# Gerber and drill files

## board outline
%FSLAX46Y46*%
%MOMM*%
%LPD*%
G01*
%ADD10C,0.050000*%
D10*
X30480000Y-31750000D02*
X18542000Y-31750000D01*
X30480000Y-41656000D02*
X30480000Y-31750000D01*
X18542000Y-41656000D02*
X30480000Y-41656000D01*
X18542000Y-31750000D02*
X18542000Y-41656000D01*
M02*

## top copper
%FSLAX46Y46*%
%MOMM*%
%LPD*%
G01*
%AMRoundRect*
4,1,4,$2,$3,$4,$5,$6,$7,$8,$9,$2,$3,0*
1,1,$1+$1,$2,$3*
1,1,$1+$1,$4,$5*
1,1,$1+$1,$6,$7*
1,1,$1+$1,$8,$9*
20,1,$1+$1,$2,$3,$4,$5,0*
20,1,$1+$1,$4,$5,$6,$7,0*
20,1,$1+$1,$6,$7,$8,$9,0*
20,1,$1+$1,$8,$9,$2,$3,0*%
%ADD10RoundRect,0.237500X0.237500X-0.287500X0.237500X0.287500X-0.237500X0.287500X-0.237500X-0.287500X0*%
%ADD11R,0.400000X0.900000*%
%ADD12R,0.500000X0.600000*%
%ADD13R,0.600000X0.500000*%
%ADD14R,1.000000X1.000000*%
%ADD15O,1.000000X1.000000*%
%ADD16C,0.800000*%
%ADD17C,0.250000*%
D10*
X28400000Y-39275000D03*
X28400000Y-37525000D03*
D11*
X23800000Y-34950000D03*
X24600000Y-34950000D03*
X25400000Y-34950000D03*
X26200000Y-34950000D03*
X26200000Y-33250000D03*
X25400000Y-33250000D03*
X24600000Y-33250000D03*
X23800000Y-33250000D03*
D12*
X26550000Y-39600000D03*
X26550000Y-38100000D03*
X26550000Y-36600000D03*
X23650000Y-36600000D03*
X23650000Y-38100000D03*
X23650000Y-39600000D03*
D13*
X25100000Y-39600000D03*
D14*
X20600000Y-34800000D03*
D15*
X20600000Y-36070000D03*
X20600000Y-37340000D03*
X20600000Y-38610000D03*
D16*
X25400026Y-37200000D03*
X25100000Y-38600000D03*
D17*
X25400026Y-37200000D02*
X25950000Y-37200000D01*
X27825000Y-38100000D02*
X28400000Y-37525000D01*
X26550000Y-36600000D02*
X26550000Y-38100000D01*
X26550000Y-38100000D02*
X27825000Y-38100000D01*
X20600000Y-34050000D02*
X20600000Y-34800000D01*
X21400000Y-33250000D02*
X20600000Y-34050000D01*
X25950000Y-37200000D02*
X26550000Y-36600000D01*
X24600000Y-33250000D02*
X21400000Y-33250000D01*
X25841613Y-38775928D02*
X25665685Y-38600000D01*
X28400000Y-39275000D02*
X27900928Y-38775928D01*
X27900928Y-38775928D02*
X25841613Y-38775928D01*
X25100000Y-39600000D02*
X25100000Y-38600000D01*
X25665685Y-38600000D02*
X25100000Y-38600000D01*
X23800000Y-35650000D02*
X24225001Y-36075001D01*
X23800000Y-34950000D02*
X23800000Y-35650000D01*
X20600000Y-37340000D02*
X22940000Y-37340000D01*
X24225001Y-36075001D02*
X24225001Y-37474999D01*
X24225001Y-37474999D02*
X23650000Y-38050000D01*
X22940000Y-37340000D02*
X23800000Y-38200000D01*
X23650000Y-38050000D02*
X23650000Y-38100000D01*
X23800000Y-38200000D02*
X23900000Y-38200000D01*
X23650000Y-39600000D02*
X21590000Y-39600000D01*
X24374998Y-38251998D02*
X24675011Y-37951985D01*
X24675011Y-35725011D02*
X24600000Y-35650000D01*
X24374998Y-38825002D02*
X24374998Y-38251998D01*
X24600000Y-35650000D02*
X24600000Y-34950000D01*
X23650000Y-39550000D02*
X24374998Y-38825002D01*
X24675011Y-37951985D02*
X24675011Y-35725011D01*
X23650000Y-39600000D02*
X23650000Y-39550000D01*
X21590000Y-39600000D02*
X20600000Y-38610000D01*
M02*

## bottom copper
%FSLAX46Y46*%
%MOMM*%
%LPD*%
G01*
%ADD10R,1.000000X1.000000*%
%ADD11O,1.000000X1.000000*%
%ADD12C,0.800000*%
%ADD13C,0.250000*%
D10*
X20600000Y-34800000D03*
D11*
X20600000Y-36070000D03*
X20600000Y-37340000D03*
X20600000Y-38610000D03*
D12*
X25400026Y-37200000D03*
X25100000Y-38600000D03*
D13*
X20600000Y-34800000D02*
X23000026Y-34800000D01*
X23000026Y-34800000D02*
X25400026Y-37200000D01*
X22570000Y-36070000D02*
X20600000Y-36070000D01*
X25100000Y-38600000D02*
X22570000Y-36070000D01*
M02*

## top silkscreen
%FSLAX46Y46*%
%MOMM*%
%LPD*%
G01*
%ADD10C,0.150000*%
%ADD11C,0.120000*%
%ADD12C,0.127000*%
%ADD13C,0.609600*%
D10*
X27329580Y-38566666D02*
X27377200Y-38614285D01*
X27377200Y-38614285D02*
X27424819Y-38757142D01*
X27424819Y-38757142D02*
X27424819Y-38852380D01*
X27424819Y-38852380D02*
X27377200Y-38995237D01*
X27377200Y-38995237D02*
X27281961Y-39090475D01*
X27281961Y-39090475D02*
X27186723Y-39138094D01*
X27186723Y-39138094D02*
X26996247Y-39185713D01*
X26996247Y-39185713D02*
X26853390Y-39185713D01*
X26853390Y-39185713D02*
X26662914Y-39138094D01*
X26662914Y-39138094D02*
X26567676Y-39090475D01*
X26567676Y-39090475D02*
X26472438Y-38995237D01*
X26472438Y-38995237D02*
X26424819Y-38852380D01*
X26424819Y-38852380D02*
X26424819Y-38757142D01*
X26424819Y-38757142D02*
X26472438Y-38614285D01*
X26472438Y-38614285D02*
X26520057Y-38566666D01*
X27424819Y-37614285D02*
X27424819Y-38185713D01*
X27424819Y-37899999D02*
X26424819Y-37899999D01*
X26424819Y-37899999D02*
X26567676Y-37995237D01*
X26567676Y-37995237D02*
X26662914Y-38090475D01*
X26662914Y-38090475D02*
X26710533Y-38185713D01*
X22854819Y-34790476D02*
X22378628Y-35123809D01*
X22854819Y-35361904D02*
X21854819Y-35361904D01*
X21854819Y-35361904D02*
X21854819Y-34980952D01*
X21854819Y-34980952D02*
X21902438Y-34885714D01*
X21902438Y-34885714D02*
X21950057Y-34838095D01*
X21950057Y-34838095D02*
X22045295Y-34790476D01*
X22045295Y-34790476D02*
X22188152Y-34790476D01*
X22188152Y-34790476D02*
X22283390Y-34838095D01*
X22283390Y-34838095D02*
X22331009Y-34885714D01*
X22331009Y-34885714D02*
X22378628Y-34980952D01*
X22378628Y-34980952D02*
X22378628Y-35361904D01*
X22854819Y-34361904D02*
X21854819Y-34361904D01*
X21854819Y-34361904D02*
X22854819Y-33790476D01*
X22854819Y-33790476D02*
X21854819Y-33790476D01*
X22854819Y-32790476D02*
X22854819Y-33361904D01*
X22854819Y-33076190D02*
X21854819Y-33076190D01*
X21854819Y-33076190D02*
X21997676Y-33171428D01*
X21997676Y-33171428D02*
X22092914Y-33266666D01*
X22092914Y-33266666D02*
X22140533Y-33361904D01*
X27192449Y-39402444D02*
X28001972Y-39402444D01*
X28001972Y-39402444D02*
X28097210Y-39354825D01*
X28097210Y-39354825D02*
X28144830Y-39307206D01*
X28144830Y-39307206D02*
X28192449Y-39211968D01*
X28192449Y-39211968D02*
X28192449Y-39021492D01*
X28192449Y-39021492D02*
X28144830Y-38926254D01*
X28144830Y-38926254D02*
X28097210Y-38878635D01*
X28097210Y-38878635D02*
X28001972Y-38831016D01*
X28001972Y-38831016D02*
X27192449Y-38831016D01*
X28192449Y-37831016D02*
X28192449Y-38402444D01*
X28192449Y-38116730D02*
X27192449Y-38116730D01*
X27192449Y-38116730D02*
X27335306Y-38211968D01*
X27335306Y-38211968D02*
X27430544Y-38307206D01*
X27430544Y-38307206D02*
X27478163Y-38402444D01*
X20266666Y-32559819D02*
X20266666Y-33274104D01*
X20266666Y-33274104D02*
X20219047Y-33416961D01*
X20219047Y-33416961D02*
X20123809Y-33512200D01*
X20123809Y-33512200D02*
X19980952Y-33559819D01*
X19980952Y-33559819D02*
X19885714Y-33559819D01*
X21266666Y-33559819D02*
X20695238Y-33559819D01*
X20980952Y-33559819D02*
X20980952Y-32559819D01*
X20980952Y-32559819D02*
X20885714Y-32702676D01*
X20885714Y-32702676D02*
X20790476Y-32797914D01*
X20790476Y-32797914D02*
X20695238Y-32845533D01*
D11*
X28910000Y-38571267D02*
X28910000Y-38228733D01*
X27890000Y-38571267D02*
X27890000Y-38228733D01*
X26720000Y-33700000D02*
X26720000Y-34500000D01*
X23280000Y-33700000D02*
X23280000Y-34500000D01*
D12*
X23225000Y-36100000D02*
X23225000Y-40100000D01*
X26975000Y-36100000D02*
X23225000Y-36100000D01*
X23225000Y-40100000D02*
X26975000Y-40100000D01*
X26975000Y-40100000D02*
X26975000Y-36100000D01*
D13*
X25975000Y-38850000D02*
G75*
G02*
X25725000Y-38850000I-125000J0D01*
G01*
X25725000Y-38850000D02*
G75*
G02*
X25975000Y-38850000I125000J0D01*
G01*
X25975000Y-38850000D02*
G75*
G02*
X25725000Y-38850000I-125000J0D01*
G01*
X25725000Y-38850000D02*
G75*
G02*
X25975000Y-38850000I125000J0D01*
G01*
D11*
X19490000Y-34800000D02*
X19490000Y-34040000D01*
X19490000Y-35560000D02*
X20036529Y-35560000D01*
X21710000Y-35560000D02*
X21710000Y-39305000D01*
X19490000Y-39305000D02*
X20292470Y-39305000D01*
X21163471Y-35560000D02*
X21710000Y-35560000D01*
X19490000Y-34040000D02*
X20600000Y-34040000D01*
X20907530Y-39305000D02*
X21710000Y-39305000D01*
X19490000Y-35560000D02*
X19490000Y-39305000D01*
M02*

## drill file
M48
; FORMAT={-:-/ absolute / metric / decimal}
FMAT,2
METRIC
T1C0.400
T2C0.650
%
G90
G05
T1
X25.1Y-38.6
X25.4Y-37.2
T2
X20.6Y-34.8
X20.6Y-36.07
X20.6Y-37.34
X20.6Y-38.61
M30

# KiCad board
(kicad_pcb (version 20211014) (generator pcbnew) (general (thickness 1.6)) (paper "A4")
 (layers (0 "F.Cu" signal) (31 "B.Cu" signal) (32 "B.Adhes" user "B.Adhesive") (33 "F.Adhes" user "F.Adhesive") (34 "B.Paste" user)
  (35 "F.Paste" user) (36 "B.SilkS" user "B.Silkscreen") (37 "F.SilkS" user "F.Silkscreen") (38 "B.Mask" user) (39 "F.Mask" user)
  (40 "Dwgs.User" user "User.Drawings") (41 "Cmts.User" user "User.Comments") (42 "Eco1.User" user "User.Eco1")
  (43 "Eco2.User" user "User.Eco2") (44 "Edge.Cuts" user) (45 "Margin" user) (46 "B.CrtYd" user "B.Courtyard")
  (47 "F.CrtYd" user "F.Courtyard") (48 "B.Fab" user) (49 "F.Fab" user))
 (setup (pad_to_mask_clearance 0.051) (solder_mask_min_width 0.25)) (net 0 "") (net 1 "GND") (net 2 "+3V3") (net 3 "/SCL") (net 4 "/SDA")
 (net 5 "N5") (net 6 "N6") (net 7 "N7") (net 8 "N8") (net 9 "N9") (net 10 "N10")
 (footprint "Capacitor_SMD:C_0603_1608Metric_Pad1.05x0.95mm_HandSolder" (layer "F.Cu") (at 28.4 38.4 90)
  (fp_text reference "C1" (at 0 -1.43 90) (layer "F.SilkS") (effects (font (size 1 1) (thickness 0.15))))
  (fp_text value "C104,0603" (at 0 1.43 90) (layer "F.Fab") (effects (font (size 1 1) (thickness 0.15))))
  (fp_line (start -0.171267 0.51) (end 0.171267 0.51) (layer "F.SilkS") (width 0.12))
  (fp_line (start -0.171267 -0.51) (end 0.171267 -0.51) (layer "F.SilkS") (width 0.12))
  (pad "1" smd roundrect locked (at -0.875 0 90) (size 1.05 0.95) (layers "F.Cu" "F.Paste" "F.Mask") (roundrect_rratio 0.25) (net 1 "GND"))
  (pad "2" smd roundrect locked (at 0.875 0 90) (size 1.05 0.95) (layers "F.Cu" "F.Paste" "F.Mask") (roundrect_rratio 0.25) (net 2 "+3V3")))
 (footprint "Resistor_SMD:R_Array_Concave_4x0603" (layer "F.Cu") (at 25 34.1 90)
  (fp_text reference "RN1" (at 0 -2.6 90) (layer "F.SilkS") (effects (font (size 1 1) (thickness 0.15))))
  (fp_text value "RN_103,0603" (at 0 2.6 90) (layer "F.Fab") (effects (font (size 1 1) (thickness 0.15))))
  (fp_line (start 0.4 1.72) (end -0.4 1.72) (layer "F.SilkS") (width 0.12))
  (fp_line (start 0.4 -1.72) (end -0.4 -1.72) (layer "F.SilkS") (width 0.12))
  (pad "1" smd rect locked (at -0.85 -1.2 90) (size 0.9 0.4) (layers "F.Cu" "F.Paste" "F.Mask") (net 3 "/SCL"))
  (pad "2" smd rect locked (at -0.85 -0.4 90) (size 0.9 0.4) (layers "F.Cu" "F.Paste" "F.Mask") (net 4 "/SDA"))
  (pad "3" smd rect locked (at -0.85 0.4 90) (size 0.9 0.4) (layers "F.Cu" "F.Paste" "F.Mask") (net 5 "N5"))
  (pad "4" smd rect locked (at -0.85 1.2 90) (size 0.9 0.4) (layers "F.Cu" "F.Paste" "F.Mask") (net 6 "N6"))
  (pad "5" smd rect locked (at 0.85 1.2 90) (size 0.9 0.4) (layers "F.Cu" "F.Paste" "F.Mask") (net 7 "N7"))
  (pad "6" smd rect locked (at 0.85 0.4 90) (size 0.9 0.4) (layers "F.Cu" "F.Paste" "F.Mask") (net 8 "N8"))
  (pad "7" smd rect locked (at 0.85 -0.4 90) (size 0.9 0.4) (layers "F.Cu" "F.Paste" "F.Mask") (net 2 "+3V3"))
  (pad "8" smd rect locked (at 0.85 -1.2 90) (size 0.9 0.4) (layers "F.Cu" "F.Paste" "F.Mask") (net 2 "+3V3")))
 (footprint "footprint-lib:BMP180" (layer "F.Cu") (at 25.1 38.1 -90)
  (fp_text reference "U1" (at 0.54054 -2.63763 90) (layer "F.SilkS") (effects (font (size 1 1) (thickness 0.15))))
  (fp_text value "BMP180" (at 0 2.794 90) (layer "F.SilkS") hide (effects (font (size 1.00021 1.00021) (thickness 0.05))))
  (fp_line (start -2 1.875) (end 2 1.875) (layer "F.SilkS") (width 0.127))
  (fp_line (start -2 -1.875) (end -2 1.875) (layer "F.SilkS") (width 0.127))
  (fp_line (start 2 1.875) (end 2 -1.875) (layer "F.SilkS") (width 0.127))
  (fp_line (start 2 -1.875) (end -2 -1.875) (layer "F.SilkS") (width 0.127))
  (fp_circle (center 0.75 -0.75) (end 0.875 -0.75) (layer "F.SilkS") (width 0.6096) (fill none))
  (fp_circle (center 0.75 -0.75) (end 0.875 -0.75) (layer "F.SilkS") (width 0.6096) (fill none))
  (pad "1" smd rect locked (at 1.5 -1.45) (size 0.5 0.6) (layers "F.Cu" "F.Paste" "F.Mask") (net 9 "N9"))
  (pad "2" smd rect locked (at 0 -1.45) (size 0.5 0.6) (layers "F.Cu" "F.Paste" "F.Mask") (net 2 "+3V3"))
  (pad "3" smd rect locked (at -1.5 -1.45) (size 0.5 0.6) (layers "F.Cu" "F.Paste" "F.Mask") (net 2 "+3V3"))
  (pad "4" smd rect locked (at -1.5 1.45) (size 0.5 0.6) (layers "F.Cu" "F.Paste" "F.Mask") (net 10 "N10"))
  (pad "5" smd rect locked (at 0 1.45) (size 0.5 0.6) (layers "F.Cu" "F.Paste" "F.Mask") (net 3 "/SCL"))
  (pad "6" smd rect locked (at 1.5 1.45) (size 0.5 0.6) (layers "F.Cu" "F.Paste" "F.Mask") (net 4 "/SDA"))
  (pad "7" smd rect locked (at 1.5 0 90) (size 0.5 0.6) (layers "F.Cu" "F.Paste" "F.Mask") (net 1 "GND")))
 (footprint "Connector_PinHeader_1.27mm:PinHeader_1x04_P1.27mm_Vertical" (layer "F.Cu") (at 20.6 34.8)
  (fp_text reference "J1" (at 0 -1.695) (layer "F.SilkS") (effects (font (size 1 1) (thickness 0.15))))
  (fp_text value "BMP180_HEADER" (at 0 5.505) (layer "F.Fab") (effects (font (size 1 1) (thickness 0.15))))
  (fp_line (start -1.11 0) (end -1.11 -0.76) (layer "F.SilkS") (width 0.12))
  (fp_line (start -1.11 0.76) (end -0.563471 0.76) (layer "F.SilkS") (width 0.12))
  (fp_line (start 1.11 0.76) (end 1.11 4.505) (layer "F.SilkS") (width 0.12))
  (fp_line (start -1.11 4.505) (end -0.30753 4.505) (layer "F.SilkS") (width 0.12))
  (fp_line (start 0.563471 0.76) (end 1.11 0.76) (layer "F.SilkS") (width 0.12))
  (fp_line (start -1.11 -0.76) (end 0 -0.76) (layer "F.SilkS") (width 0.12))
  (fp_line (start 0.30753 4.505) (end 1.11 4.505) (layer "F.SilkS") (width 0.12))
  (fp_line (start -1.11 0.76) (end -1.11 4.505) (layer "F.SilkS") (width 0.12))
  (pad "1" thru_hole rect locked (at 0 0) (size 1 1) (drill 0.65) (layers *.Cu *.Mask) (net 2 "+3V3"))
  (pad "2" thru_hole oval locked (at 0 1.27) (size 1 1) (drill 0.65) (layers *.Cu *.Mask) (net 1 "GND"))
  (pad "3" thru_hole oval locked (at 0 2.54) (size 1 1) (drill 0.65) (layers *.Cu *.Mask) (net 3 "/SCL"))
  (pad "4" thru_hole oval locked (at 0 3.81) (size 1 1) (drill 0.65) (layers *.Cu *.Mask) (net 4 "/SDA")))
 (gr_line (start 30.48 31.75) (end 18.542 31.75) (layer "Edge.Cuts") (width 0.05))
 (gr_line (start 30.48 41.656) (end 30.48 31.75) (layer "Edge.Cuts") (width 0.05))
 (gr_line (start 18.542 41.656) (end 30.48 41.656) (layer "Edge.Cuts") (width 0.05))
 (gr_line (start 18.542 31.75) (end 18.542 41.656) (layer "Edge.Cuts") (width 0.05))
 (segment (start 25.400026 37.2) (end 25.95 37.2) (width 0.25) (layer "F.Cu") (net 2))
 (segment (start 27.825 38.1) (end 28.4 37.525) (width 0.25) (layer "F.Cu") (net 2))
 (segment (start 26.55 36.6) (end 26.55 38.1) (width 0.25) (layer "F.Cu") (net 2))
 (segment (start 26.55 38.1) (end 27.825 38.1) (width 0.25) (layer "F.Cu") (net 2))
 (segment (start 20.6 34.05) (end 20.6 34.8) (width 0.25) (layer "F.Cu") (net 2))
 (segment (start 21.4 33.25) (end 20.6 34.05) (width 0.25) (layer "F.Cu") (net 2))
 (segment (start 25.95 37.2) (end 26.55 36.6) (width 0.25) (layer "F.Cu") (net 2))
 (segment (start 24.6 33.25) (end 21.4 33.25) (width 0.25) (layer "F.Cu") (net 2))
 (via (at 25.400026 37.2) (size 0.8) (drill 0.4) (layers "F.Cu" "B.Cu") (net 2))
 (segment (start 20.6 34.8) (end 23.000026 34.8) (width 0.25) (layer "B.Cu") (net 2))
 (segment (start 23.000026 34.8) (end 25.400026 37.2) (width 0.25) (layer "B.Cu") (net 2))
 (segment (start 25.841613 38.775928) (end 25.665685 38.6) (width 0.25) (layer "F.Cu") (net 1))
 (segment (start 28.4 39.275) (end 27.900928 38.775928) (width 0.25) (layer "F.Cu") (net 1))
 (segment (start 27.900928 38.775928) (end 25.841613 38.775928) (width 0.25) (layer "F.Cu") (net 1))
 (segment (start 25.1 39.6) (end 25.1 38.6) (width 0.25) (layer "F.Cu") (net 1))
 (segment (start 25.665685 38.6) (end 25.1 38.6) (width 0.25) (layer "F.Cu") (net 1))
 (via (at 25.1 38.6) (size 0.8) (drill 0.4) (layers "F.Cu" "B.Cu") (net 1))
 (segment (start 22.57 36.07) (end 20.6 36.07) (width 0.25) (layer "B.Cu") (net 1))
 (segment (start 25.1 38.6) (end 22.57 36.07) (width 0.25) (layer "B.Cu") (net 1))
 (segment (start 23.8 35.65) (end 24.225001 36.075001) (width 0.25) (layer "F.Cu") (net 3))
 (segment (start 23.8 34.95) (end 23.8 35.65) (width 0.25) (layer "F.Cu") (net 3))
 (segment (start 20.6 37.34) (end 22.94 37.34) (width 0.25) (layer "F.Cu") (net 3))
 (segment (start 24.225001 36.075001) (end 24.225001 37.474999) (width 0.25) (layer "F.Cu") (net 3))
 (segment (start 24.225001 37.474999) (end 23.65 38.05) (width 0.25) (layer "F.Cu") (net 3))
 (segment (start 22.94 37.34) (end 23.8 38.2) (width 0.25) (layer "F.Cu") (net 3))
 (segment (start 23.65 38.05) (end 23.65 38.1) (width 0.25) (layer "F.Cu") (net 3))
 (segment (start 23.8 38.2) (end 23.9 38.2) (width 0.25) (layer "F.Cu") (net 3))
 (segment (start 23.65 39.6) (end 21.59 39.6) (width 0.25) (layer "F.Cu") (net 4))
 (segment (start 24.374998 38.251998) (end 24.675011 37.951985) (width 0.25) (layer "F.Cu") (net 4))
 (segment (start 24.675011 35.725011) (end 24.6 35.65) (width 0.25) (layer "F.Cu") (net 4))
 (segment (start 24.374998 38.825002) (end 24.374998 38.251998) (width 0.25) (layer "F.Cu") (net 4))
 (segment (start 24.6 35.65) (end 24.6 34.95) (width 0.25) (layer "F.Cu") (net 4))
 (segment (start 23.65 39.55) (end 24.374998 38.825002) (width 0.25) (layer "F.Cu") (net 4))
 (segment (start 24.675011 37.951985) (end 24.675011 35.725011) (width 0.25) (layer "F.Cu") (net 4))
 (segment (start 23.65 39.6) (end 23.65 39.55) (width 0.25) (layer "F.Cu") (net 4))
 (segment (start 21.59 39.6) (end 20.6 38.61) (width 0.25) (layer "F.Cu") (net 4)))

